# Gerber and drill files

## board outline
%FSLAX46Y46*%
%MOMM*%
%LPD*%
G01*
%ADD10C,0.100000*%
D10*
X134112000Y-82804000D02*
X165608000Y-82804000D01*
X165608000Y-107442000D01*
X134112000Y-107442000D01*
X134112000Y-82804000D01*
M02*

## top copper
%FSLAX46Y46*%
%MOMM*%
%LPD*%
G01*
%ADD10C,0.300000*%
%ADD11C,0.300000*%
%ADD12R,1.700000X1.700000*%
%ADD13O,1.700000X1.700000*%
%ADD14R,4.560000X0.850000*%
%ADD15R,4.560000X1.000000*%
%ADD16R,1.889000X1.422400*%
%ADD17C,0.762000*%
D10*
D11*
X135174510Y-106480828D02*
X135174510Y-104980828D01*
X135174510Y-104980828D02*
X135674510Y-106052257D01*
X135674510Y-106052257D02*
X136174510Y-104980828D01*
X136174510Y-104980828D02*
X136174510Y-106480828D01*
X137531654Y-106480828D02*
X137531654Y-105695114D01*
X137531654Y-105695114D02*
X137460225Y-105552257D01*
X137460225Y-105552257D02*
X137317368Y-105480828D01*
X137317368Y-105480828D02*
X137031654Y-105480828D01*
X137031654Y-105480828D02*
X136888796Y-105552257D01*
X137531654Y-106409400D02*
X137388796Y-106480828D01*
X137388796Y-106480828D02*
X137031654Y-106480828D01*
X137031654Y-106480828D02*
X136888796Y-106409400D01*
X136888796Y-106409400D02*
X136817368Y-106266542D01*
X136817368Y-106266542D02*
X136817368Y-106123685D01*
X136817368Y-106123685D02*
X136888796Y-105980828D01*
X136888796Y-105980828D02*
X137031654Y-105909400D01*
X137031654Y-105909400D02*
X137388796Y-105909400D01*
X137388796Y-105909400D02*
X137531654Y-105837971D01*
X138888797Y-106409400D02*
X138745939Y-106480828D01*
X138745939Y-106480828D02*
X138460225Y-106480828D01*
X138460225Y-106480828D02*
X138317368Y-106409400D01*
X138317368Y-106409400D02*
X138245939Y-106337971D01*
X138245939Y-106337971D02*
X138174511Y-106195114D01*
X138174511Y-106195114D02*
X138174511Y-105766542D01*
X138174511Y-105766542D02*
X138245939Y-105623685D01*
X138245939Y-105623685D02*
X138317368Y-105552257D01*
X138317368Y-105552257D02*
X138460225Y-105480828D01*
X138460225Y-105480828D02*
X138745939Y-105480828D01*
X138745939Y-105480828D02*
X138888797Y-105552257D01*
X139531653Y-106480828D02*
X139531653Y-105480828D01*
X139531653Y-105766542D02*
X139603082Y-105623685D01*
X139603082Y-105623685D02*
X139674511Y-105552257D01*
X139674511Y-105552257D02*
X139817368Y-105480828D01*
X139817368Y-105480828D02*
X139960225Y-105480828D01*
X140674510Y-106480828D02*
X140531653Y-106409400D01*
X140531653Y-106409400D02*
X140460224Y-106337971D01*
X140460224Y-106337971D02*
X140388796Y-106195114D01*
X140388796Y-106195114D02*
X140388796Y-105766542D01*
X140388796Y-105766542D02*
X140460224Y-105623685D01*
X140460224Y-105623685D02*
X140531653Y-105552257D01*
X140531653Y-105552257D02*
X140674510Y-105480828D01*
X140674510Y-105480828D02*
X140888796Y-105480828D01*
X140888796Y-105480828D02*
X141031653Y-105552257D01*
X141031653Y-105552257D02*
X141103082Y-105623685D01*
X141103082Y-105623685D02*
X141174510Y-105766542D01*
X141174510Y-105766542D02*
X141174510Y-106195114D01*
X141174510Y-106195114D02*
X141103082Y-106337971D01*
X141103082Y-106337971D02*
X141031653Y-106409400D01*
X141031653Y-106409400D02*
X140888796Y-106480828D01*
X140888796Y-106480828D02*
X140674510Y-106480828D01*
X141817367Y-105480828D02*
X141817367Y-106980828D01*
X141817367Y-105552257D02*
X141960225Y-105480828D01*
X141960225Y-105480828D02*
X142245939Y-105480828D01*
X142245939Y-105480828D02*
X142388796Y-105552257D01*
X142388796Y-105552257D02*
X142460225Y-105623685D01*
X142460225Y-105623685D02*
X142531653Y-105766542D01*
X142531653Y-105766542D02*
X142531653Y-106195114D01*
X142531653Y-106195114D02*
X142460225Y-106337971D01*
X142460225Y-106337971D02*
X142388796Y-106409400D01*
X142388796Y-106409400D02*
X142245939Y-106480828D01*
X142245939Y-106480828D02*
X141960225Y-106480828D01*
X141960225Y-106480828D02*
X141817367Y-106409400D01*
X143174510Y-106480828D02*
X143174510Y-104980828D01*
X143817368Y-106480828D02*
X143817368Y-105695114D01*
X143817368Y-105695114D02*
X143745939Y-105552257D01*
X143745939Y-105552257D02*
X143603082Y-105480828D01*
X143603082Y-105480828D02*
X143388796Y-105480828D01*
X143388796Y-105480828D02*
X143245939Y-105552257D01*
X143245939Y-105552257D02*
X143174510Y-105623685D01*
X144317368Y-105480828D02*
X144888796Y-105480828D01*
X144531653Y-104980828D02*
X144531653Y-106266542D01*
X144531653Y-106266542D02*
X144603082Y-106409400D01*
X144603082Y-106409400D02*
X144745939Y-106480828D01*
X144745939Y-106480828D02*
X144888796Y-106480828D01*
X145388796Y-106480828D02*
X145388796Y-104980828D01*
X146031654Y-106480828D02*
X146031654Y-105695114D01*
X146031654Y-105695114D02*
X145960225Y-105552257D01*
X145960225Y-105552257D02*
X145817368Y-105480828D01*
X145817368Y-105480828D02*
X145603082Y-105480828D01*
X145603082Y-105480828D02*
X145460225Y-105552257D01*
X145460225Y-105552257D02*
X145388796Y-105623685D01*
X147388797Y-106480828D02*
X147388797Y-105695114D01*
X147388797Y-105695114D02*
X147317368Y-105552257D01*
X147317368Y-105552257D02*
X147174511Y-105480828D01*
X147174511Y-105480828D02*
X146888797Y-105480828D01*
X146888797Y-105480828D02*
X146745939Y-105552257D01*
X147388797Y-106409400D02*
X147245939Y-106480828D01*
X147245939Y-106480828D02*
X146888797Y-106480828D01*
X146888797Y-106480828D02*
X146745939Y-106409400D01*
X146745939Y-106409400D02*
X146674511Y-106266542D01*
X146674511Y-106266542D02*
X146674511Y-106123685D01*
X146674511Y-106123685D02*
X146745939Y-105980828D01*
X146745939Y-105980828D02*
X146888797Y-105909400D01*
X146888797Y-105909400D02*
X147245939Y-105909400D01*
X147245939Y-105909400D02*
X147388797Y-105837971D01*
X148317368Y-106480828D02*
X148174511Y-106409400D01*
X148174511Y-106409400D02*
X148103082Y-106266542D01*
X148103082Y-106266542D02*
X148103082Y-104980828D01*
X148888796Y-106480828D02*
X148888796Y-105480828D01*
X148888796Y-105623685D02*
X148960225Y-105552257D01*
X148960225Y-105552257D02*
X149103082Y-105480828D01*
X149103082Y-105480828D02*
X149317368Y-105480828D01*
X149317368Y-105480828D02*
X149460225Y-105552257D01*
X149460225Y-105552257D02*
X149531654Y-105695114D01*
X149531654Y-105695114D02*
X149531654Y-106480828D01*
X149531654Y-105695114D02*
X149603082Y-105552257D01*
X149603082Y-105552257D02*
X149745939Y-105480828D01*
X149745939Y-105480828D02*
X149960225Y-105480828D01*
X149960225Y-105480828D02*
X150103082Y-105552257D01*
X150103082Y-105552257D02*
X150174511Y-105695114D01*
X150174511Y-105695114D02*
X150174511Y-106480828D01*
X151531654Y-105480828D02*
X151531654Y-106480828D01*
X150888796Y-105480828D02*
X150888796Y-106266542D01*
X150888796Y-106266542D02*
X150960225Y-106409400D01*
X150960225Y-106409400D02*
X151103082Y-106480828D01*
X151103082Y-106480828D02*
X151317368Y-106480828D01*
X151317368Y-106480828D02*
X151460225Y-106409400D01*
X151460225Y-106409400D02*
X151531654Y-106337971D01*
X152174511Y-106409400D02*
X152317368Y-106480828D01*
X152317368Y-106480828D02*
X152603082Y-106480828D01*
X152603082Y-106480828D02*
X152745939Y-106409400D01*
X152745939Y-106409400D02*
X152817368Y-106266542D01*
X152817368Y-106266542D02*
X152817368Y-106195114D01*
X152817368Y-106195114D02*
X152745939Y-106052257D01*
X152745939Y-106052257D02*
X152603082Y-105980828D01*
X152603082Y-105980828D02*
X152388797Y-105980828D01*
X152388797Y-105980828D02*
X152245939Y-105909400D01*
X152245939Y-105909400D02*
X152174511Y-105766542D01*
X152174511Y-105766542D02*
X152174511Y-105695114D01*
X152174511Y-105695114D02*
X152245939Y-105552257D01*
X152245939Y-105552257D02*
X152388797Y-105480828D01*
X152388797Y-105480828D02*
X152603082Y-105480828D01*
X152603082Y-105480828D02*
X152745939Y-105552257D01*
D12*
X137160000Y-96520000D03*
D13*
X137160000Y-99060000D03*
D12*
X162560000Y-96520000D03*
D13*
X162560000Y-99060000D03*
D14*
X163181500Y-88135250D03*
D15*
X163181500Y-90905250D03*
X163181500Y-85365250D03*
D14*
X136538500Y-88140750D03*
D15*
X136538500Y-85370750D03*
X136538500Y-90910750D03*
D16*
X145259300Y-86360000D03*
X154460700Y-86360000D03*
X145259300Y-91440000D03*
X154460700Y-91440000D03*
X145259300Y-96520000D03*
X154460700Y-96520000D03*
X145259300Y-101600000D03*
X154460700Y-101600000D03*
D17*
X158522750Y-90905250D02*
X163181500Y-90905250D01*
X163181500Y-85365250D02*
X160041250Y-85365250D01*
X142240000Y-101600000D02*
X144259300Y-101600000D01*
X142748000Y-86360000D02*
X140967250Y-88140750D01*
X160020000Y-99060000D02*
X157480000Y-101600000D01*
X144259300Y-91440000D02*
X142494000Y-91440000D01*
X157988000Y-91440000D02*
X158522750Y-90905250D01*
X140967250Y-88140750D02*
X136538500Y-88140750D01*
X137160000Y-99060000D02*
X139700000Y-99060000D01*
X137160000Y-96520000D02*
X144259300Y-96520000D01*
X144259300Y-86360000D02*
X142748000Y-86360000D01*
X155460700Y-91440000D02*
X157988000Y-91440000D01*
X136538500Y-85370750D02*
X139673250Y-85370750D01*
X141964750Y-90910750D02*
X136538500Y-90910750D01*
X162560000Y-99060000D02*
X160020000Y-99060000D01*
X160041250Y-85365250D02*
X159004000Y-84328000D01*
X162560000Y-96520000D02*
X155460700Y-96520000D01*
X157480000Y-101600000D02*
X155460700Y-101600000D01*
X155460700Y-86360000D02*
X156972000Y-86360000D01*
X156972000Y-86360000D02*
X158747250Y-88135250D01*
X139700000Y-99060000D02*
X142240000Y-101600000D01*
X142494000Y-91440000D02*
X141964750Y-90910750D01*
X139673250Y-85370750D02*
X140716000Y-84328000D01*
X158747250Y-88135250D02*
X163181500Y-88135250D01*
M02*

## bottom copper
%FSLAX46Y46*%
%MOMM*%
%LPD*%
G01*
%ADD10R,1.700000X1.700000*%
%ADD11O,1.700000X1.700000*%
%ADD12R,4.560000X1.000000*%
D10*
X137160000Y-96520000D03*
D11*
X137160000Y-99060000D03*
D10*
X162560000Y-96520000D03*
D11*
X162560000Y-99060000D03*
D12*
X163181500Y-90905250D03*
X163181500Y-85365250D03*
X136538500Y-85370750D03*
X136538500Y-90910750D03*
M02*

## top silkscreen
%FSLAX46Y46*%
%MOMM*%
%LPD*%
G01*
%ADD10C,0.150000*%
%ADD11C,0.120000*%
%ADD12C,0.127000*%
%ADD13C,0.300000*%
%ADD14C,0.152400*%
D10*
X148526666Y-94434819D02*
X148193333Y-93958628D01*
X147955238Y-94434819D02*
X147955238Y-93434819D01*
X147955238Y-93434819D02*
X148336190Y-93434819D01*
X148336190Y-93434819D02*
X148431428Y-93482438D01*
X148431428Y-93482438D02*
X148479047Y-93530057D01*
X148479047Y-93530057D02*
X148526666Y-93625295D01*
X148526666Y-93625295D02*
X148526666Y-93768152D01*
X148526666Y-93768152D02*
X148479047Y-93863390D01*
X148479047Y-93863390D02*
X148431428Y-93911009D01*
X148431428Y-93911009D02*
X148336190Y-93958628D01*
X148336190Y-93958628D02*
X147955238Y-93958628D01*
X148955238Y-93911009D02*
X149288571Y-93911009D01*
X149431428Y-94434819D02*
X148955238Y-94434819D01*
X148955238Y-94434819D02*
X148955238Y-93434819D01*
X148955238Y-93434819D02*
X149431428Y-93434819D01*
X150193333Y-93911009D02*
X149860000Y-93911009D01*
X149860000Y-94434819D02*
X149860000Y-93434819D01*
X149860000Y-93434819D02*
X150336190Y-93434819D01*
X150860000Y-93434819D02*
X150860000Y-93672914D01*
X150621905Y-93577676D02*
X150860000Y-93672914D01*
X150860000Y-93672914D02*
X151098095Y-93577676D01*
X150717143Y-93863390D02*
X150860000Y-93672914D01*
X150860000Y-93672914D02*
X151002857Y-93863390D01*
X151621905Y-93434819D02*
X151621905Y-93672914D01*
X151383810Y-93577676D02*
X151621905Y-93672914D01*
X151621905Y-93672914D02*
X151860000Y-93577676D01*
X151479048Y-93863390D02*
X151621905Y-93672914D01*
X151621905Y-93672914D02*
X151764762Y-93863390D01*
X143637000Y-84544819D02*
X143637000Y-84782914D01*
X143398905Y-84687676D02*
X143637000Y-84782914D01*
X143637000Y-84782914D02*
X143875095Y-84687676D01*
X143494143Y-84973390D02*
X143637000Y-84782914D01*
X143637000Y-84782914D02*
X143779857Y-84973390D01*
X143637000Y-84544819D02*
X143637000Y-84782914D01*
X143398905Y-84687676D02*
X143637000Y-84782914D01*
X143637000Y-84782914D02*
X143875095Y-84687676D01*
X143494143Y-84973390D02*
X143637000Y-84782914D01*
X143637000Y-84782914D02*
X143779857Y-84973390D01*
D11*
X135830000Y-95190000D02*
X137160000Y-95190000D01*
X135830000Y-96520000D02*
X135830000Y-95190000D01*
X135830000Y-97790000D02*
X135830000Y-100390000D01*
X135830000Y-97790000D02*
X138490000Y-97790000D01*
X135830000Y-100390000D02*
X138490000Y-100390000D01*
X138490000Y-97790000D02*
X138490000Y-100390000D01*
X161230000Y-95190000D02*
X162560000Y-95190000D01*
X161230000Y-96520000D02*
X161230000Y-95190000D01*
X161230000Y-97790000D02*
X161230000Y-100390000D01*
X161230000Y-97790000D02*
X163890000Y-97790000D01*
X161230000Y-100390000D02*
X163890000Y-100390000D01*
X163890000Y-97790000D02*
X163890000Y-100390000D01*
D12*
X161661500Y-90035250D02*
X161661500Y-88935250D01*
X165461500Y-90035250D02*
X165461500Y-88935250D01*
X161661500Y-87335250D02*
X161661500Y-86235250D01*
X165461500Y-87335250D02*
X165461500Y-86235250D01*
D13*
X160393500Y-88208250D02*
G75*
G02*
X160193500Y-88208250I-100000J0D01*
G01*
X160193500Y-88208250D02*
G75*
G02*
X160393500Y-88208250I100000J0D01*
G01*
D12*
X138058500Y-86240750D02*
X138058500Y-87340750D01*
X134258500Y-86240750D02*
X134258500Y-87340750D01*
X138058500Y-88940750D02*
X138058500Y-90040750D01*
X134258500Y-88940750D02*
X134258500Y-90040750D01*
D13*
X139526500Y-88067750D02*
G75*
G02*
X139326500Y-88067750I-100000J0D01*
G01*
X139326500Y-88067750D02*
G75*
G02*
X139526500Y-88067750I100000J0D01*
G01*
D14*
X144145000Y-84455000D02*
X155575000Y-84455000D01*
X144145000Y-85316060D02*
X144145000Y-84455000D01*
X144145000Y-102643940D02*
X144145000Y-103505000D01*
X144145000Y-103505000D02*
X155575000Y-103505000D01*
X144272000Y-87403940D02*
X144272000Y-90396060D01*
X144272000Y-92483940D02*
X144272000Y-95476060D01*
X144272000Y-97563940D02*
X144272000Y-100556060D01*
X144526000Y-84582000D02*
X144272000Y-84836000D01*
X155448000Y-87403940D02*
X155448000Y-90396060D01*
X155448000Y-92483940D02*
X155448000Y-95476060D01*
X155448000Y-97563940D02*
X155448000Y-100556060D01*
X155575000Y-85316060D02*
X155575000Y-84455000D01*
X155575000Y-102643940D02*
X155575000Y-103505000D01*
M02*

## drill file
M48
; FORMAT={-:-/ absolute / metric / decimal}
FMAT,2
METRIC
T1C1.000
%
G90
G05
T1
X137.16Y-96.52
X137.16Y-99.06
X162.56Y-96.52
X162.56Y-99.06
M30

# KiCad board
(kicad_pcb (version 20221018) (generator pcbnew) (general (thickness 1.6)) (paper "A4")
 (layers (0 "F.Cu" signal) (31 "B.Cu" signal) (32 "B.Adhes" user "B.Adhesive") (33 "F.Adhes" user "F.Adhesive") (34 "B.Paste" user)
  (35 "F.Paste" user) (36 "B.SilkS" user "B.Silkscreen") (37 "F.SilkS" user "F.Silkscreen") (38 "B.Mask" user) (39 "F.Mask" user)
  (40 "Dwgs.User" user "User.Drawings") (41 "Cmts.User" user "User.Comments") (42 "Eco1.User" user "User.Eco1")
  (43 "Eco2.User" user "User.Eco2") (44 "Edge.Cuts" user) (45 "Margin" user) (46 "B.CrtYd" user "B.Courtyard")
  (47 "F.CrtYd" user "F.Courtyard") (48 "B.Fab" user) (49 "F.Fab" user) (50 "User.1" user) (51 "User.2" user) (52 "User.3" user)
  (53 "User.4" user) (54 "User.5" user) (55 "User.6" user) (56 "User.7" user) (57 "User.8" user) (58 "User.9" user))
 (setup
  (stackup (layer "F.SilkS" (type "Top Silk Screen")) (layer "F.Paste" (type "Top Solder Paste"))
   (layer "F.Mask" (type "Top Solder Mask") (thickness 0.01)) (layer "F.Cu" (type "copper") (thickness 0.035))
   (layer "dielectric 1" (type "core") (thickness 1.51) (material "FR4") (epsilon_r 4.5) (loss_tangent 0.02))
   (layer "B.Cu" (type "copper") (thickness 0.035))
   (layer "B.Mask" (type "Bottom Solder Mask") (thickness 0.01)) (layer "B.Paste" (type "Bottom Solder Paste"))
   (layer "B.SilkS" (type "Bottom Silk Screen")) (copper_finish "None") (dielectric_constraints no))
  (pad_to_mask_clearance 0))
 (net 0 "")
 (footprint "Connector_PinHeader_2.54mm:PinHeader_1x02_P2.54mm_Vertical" (layer "F.Cu") (at 137.16 96.52)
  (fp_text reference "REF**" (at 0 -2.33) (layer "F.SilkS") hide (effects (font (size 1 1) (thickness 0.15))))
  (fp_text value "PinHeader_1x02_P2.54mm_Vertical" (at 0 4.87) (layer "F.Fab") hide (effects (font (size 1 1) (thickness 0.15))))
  (fp_line (start -1.33 -1.33) (end 0 -1.33) (stroke (width 0.12) (type solid)) (layer "F.SilkS"))
  (fp_line (start -1.33 0) (end -1.33 -1.33) (stroke (width 0.12) (type solid)) (layer "F.SilkS"))
  (fp_line (start -1.33 1.27) (end -1.33 3.87) (stroke (width 0.12) (type solid)) (layer "F.SilkS"))
  (fp_line (start -1.33 1.27) (end 1.33 1.27) (stroke (width 0.12) (type solid)) (layer "F.SilkS"))
  (fp_line (start -1.33 3.87) (end 1.33 3.87) (stroke (width 0.12) (type solid)) (layer "F.SilkS"))
  (fp_line (start 1.33 1.27) (end 1.33 3.87) (stroke (width 0.12) (type solid)) (layer "F.SilkS"))
  (pad "1" thru_hole rect (at 0 0) (size 1.7 1.7) (drill 1) (layers "*.Cu" "*.Mask"))
  (pad "2" thru_hole oval (at 0 2.54) (size 1.7 1.7) (drill 1) (layers "*.Cu" "*.Mask")))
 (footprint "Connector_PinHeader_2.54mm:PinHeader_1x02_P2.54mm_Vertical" (layer "F.Cu") (at 162.56 96.52)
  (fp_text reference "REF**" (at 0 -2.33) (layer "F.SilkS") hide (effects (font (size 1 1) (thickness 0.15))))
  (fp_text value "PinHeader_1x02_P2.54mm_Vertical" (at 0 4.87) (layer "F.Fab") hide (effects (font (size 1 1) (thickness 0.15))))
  (fp_line (start -1.33 -1.33) (end 0 -1.33) (stroke (width 0.12) (type solid)) (layer "F.SilkS"))
  (fp_line (start -1.33 0) (end -1.33 -1.33) (stroke (width 0.12) (type solid)) (layer "F.SilkS"))
  (fp_line (start -1.33 1.27) (end -1.33 3.87) (stroke (width 0.12) (type solid)) (layer "F.SilkS"))
  (fp_line (start -1.33 1.27) (end 1.33 1.27) (stroke (width 0.12) (type solid)) (layer "F.SilkS"))
  (fp_line (start -1.33 3.87) (end 1.33 3.87) (stroke (width 0.12) (type solid)) (layer "F.SilkS"))
  (fp_line (start 1.33 1.27) (end 1.33 3.87) (stroke (width 0.12) (type solid)) (layer "F.SilkS"))
  (pad "1" thru_hole rect (at 0 0) (size 1.7 1.7) (drill 1) (layers "*.Cu" "*.Mask"))
  (pad "2" thru_hole oval (at 0 2.54) (size 1.7 1.7) (drill 1) (layers "*.Cu" "*.Mask")))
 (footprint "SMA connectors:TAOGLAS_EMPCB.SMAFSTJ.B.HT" (layer "F.Cu") (at 163.1815 88.13525 90)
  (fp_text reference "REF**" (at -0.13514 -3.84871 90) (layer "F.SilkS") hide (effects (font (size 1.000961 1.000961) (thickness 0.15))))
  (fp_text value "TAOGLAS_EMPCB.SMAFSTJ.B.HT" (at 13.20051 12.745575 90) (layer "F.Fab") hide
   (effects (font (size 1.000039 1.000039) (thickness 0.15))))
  (fp_line (start -1.9 -1.52) (end -0.8 -1.52) (stroke (width 0.127) (type solid)) (layer "F.SilkS"))
  (fp_line (start -1.9 2.28) (end -0.8 2.28) (stroke (width 0.127) (type solid)) (layer "F.SilkS"))
  (fp_line (start 0.8 -1.52) (end 1.9 -1.52) (stroke (width 0.127) (type solid)) (layer "F.SilkS"))
  (fp_line (start 0.8 2.28) (end 1.9 2.28) (stroke (width 0.127) (type solid)) (layer "F.SilkS"))
  (fp_circle (center -0.073 -2.888) (end 0.027 -2.888) (stroke (width 0.3) (type solid)) (fill none) (layer "F.SilkS"))
  (pad "1" smd rect (at 0 0 90) (size 0.85 4.56) (layers "F.Cu" "F.Paste" "F.Mask") (solder_mask_margin 0.102))
  (pad "SH1" smd rect (at -2.77 0 90) (size 1 4.56) (layers "F.Cu" "F.Paste" "F.Mask") (solder_mask_margin 0.102))
  (pad "SH2" smd rect (at 2.77 0 90) (size 1 4.56) (layers "F.Cu" "F.Paste" "F.Mask") (solder_mask_margin 0.102))
  (pad "SH3" smd rect (at -2.77 0 90) (size 1 4.56) (layers "B.Cu" "B.Paste" "B.Mask") (solder_mask_margin 0.102))
  (pad "SH4" smd rect (at 2.77 0 90) (size 1 4.56) (layers "B.Cu" "B.Paste" "B.Mask") (solder_mask_margin 0.102)))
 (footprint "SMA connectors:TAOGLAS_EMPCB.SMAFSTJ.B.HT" (layer "F.Cu") (at 136.5385 88.14075 -90)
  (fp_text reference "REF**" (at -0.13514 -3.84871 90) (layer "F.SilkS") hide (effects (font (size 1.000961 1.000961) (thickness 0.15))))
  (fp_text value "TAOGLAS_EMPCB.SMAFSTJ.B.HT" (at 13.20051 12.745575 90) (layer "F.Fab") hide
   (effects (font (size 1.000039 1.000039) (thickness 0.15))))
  (fp_line (start -1.9 -1.52) (end -0.8 -1.52) (stroke (width 0.127) (type solid)) (layer "F.SilkS"))
  (fp_line (start -1.9 2.28) (end -0.8 2.28) (stroke (width 0.127) (type solid)) (layer "F.SilkS"))
  (fp_line (start 0.8 -1.52) (end 1.9 -1.52) (stroke (width 0.127) (type solid)) (layer "F.SilkS"))
  (fp_line (start 0.8 2.28) (end 1.9 2.28) (stroke (width 0.127) (type solid)) (layer "F.SilkS"))
  (fp_circle (center -0.073 -2.888) (end 0.027 -2.888) (stroke (width 0.3) (type solid)) (fill none) (layer "F.SilkS"))
  (pad "1" smd rect (at 0 0 270) (size 0.85 4.56) (layers "F.Cu" "F.Paste" "F.Mask") (solder_mask_margin 0.102))
  (pad "SH1" smd rect (at -2.77 0 270) (size 1 4.56) (layers "F.Cu" "F.Paste" "F.Mask") (solder_mask_margin 0.102))
  (pad "SH2" smd rect (at 2.77 0 270) (size 1 4.56) (layers "F.Cu" "F.Paste" "F.Mask") (solder_mask_margin 0.102))
  (pad "SH3" smd rect (at -2.77 0 270) (size 1 4.56) (layers "B.Cu" "B.Paste" "B.Mask") (solder_mask_margin 0.102))
  (pad "SH4" smd rect (at 2.77 0 270) (size 1 4.56) (layers "B.Cu" "B.Paste" "B.Mask") (solder_mask_margin 0.102)))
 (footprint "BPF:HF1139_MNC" (layer "F.Cu") (at 149.86 93.98)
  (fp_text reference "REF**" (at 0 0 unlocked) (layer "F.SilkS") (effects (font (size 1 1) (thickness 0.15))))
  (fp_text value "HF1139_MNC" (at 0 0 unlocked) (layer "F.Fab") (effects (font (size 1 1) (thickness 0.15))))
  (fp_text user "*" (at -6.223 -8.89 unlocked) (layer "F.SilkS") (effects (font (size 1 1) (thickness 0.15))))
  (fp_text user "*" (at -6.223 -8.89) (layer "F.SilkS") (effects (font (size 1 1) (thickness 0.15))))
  (fp_line (start -5.715 -9.525) (end 5.715 -9.525) (stroke (width 0.1524) (type solid)) (layer "F.SilkS"))
  (fp_line (start -5.715 -8.66394) (end -5.715 -9.525) (stroke (width 0.1524) (type solid)) (layer "F.SilkS"))
  (fp_line (start -5.715 8.66394) (end -5.715 9.525) (stroke (width 0.1524) (type solid)) (layer "F.SilkS"))
  (fp_line (start -5.715 9.525) (end 5.715 9.525) (stroke (width 0.1524) (type solid)) (layer "F.SilkS"))
  (fp_line (start -5.588 -6.57606) (end -5.588 -3.58394) (stroke (width 0.1524) (type solid)) (layer "F.SilkS"))
  (fp_line (start -5.588 -1.49606) (end -5.588 1.49606) (stroke (width 0.1524) (type solid)) (layer "F.SilkS"))
  (fp_line (start -5.588 3.58394) (end -5.588 6.57606) (stroke (width 0.1524) (type solid)) (layer "F.SilkS"))
  (fp_line (start -5.334 -9.398) (end -5.588 -9.144) (stroke (width 0.1524) (type solid)) (layer "F.SilkS"))
  (fp_line (start 5.588 -6.57606) (end 5.588 -3.58394) (stroke (width 0.1524) (type solid)) (layer "F.SilkS"))
  (fp_line (start 5.588 -1.49606) (end 5.588 1.49606) (stroke (width 0.1524) (type solid)) (layer "F.SilkS"))
  (fp_line (start 5.588 3.58394) (end 5.588 6.57606) (stroke (width 0.1524) (type solid)) (layer "F.SilkS"))
  (fp_line (start 5.715 -8.66394) (end 5.715 -9.525) (stroke (width 0.1524) (type solid)) (layer "F.SilkS"))
  (fp_line (start 5.715 8.66394) (end 5.715 9.525) (stroke (width 0.1524) (type solid)) (layer "F.SilkS"))
  (pad "1" smd rect (at -4.6007 -7.62) (size 1.889 1.4224) (layers "F.Cu" "F.Paste" "F.Mask"))
  (pad "2" smd rect (at 4.6007 -7.62) (size 1.889 1.4224) (layers "F.Cu" "F.Paste" "F.Mask"))
  (pad "3" smd rect (at -4.6007 -2.54) (size 1.889 1.4224) (layers "F.Cu" "F.Paste" "F.Mask"))
  (pad "4" smd rect (at 4.6007 -2.54) (size 1.889 1.4224) (layers "F.Cu" "F.Paste" "F.Mask"))
  (pad "5" smd rect (at -4.6007 2.54) (size 1.889 1.4224) (layers "F.Cu" "F.Paste" "F.Mask"))
  (pad "6" smd rect (at 4.6007 2.54) (size 1.889 1.4224) (layers "F.Cu" "F.Paste" "F.Mask"))
  (pad "7" smd rect (at -4.6007 7.62) (size 1.889 1.4224) (layers "F.Cu" "F.Paste" "F.Mask"))
  (pad "8" smd rect (at 4.6007 7.62) (size 1.889 1.4224) (layers "F.Cu" "F.Paste" "F.Mask")))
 (gr_rect (start 134.112 82.804) (end 165.608 107.442) (stroke (width 0.1) (type default)) (fill none) (layer "Edge.Cuts"))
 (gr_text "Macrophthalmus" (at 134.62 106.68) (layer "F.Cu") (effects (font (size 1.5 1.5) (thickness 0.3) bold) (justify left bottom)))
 (segment (start 158.52275 90.90525) (end 163.1815 90.90525) (width 0.762) (layer "F.Cu") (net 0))
 (segment (start 163.1815 85.36525) (end 160.04125 85.36525) (width 0.762) (layer "F.Cu") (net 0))
 (segment (start 142.24 101.6) (end 144.2593 101.6) (width 0.762) (layer "F.Cu") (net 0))
 (segment (start 142.748 86.36) (end 140.96725 88.14075) (width 0.762) (layer "F.Cu") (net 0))
 (segment (start 160.02 99.06) (end 157.48 101.6) (width 0.762) (layer "F.Cu") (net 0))
 (segment (start 144.2593 91.44) (end 142.494 91.44) (width 0.762) (layer "F.Cu") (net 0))
 (segment (start 157.988 91.44) (end 158.52275 90.90525) (width 0.762) (layer "F.Cu") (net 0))
 (segment (start 140.96725 88.14075) (end 136.5385 88.14075) (width 0.762) (layer "F.Cu") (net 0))
 (segment (start 137.16 99.06) (end 139.7 99.06) (width 0.762) (layer "F.Cu") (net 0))
 (segment (start 137.16 96.52) (end 144.2593 96.52) (width 0.762) (layer "F.Cu") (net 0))
 (segment (start 144.2593 86.36) (end 142.748 86.36) (width 0.762) (layer "F.Cu") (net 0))
 (segment (start 155.4607 91.44) (end 157.988 91.44) (width 0.762) (layer "F.Cu") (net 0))
 (segment (start 136.5385 85.37075) (end 139.67325 85.37075) (width 0.762) (layer "F.Cu") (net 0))
 (segment (start 141.96475 90.91075) (end 136.5385 90.91075) (width 0.762) (layer "F.Cu") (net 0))
 (segment (start 162.56 99.06) (end 160.02 99.06) (width 0.762) (layer "F.Cu") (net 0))
 (segment (start 160.04125 85.36525) (end 159.004 84.328) (width 0.762) (layer "F.Cu") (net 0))
 (segment (start 162.56 96.52) (end 155.4607 96.52) (width 0.762) (layer "F.Cu") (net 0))
 (segment (start 157.48 101.6) (end 155.4607 101.6) (width 0.762) (layer "F.Cu") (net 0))
 (segment (start 155.4607 86.36) (end 156.972 86.36) (width 0.762) (layer "F.Cu") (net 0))
 (segment (start 156.972 86.36) (end 158.74725 88.13525) (width 0.762) (layer "F.Cu") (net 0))
 (segment (start 139.7 99.06) (end 142.24 101.6) (width 0.762) (layer "F.Cu") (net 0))
 (segment (start 142.494 91.44) (end 141.96475 90.91075) (width 0.762) (layer "F.Cu") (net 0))
 (segment (start 139.67325 85.37075) (end 140.716 84.328) (width 0.762) (layer "F.Cu") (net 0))
 (segment (start 158.74725 88.13525) (end 163.1815 88.13525) (width 0.762) (layer "F.Cu") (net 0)))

